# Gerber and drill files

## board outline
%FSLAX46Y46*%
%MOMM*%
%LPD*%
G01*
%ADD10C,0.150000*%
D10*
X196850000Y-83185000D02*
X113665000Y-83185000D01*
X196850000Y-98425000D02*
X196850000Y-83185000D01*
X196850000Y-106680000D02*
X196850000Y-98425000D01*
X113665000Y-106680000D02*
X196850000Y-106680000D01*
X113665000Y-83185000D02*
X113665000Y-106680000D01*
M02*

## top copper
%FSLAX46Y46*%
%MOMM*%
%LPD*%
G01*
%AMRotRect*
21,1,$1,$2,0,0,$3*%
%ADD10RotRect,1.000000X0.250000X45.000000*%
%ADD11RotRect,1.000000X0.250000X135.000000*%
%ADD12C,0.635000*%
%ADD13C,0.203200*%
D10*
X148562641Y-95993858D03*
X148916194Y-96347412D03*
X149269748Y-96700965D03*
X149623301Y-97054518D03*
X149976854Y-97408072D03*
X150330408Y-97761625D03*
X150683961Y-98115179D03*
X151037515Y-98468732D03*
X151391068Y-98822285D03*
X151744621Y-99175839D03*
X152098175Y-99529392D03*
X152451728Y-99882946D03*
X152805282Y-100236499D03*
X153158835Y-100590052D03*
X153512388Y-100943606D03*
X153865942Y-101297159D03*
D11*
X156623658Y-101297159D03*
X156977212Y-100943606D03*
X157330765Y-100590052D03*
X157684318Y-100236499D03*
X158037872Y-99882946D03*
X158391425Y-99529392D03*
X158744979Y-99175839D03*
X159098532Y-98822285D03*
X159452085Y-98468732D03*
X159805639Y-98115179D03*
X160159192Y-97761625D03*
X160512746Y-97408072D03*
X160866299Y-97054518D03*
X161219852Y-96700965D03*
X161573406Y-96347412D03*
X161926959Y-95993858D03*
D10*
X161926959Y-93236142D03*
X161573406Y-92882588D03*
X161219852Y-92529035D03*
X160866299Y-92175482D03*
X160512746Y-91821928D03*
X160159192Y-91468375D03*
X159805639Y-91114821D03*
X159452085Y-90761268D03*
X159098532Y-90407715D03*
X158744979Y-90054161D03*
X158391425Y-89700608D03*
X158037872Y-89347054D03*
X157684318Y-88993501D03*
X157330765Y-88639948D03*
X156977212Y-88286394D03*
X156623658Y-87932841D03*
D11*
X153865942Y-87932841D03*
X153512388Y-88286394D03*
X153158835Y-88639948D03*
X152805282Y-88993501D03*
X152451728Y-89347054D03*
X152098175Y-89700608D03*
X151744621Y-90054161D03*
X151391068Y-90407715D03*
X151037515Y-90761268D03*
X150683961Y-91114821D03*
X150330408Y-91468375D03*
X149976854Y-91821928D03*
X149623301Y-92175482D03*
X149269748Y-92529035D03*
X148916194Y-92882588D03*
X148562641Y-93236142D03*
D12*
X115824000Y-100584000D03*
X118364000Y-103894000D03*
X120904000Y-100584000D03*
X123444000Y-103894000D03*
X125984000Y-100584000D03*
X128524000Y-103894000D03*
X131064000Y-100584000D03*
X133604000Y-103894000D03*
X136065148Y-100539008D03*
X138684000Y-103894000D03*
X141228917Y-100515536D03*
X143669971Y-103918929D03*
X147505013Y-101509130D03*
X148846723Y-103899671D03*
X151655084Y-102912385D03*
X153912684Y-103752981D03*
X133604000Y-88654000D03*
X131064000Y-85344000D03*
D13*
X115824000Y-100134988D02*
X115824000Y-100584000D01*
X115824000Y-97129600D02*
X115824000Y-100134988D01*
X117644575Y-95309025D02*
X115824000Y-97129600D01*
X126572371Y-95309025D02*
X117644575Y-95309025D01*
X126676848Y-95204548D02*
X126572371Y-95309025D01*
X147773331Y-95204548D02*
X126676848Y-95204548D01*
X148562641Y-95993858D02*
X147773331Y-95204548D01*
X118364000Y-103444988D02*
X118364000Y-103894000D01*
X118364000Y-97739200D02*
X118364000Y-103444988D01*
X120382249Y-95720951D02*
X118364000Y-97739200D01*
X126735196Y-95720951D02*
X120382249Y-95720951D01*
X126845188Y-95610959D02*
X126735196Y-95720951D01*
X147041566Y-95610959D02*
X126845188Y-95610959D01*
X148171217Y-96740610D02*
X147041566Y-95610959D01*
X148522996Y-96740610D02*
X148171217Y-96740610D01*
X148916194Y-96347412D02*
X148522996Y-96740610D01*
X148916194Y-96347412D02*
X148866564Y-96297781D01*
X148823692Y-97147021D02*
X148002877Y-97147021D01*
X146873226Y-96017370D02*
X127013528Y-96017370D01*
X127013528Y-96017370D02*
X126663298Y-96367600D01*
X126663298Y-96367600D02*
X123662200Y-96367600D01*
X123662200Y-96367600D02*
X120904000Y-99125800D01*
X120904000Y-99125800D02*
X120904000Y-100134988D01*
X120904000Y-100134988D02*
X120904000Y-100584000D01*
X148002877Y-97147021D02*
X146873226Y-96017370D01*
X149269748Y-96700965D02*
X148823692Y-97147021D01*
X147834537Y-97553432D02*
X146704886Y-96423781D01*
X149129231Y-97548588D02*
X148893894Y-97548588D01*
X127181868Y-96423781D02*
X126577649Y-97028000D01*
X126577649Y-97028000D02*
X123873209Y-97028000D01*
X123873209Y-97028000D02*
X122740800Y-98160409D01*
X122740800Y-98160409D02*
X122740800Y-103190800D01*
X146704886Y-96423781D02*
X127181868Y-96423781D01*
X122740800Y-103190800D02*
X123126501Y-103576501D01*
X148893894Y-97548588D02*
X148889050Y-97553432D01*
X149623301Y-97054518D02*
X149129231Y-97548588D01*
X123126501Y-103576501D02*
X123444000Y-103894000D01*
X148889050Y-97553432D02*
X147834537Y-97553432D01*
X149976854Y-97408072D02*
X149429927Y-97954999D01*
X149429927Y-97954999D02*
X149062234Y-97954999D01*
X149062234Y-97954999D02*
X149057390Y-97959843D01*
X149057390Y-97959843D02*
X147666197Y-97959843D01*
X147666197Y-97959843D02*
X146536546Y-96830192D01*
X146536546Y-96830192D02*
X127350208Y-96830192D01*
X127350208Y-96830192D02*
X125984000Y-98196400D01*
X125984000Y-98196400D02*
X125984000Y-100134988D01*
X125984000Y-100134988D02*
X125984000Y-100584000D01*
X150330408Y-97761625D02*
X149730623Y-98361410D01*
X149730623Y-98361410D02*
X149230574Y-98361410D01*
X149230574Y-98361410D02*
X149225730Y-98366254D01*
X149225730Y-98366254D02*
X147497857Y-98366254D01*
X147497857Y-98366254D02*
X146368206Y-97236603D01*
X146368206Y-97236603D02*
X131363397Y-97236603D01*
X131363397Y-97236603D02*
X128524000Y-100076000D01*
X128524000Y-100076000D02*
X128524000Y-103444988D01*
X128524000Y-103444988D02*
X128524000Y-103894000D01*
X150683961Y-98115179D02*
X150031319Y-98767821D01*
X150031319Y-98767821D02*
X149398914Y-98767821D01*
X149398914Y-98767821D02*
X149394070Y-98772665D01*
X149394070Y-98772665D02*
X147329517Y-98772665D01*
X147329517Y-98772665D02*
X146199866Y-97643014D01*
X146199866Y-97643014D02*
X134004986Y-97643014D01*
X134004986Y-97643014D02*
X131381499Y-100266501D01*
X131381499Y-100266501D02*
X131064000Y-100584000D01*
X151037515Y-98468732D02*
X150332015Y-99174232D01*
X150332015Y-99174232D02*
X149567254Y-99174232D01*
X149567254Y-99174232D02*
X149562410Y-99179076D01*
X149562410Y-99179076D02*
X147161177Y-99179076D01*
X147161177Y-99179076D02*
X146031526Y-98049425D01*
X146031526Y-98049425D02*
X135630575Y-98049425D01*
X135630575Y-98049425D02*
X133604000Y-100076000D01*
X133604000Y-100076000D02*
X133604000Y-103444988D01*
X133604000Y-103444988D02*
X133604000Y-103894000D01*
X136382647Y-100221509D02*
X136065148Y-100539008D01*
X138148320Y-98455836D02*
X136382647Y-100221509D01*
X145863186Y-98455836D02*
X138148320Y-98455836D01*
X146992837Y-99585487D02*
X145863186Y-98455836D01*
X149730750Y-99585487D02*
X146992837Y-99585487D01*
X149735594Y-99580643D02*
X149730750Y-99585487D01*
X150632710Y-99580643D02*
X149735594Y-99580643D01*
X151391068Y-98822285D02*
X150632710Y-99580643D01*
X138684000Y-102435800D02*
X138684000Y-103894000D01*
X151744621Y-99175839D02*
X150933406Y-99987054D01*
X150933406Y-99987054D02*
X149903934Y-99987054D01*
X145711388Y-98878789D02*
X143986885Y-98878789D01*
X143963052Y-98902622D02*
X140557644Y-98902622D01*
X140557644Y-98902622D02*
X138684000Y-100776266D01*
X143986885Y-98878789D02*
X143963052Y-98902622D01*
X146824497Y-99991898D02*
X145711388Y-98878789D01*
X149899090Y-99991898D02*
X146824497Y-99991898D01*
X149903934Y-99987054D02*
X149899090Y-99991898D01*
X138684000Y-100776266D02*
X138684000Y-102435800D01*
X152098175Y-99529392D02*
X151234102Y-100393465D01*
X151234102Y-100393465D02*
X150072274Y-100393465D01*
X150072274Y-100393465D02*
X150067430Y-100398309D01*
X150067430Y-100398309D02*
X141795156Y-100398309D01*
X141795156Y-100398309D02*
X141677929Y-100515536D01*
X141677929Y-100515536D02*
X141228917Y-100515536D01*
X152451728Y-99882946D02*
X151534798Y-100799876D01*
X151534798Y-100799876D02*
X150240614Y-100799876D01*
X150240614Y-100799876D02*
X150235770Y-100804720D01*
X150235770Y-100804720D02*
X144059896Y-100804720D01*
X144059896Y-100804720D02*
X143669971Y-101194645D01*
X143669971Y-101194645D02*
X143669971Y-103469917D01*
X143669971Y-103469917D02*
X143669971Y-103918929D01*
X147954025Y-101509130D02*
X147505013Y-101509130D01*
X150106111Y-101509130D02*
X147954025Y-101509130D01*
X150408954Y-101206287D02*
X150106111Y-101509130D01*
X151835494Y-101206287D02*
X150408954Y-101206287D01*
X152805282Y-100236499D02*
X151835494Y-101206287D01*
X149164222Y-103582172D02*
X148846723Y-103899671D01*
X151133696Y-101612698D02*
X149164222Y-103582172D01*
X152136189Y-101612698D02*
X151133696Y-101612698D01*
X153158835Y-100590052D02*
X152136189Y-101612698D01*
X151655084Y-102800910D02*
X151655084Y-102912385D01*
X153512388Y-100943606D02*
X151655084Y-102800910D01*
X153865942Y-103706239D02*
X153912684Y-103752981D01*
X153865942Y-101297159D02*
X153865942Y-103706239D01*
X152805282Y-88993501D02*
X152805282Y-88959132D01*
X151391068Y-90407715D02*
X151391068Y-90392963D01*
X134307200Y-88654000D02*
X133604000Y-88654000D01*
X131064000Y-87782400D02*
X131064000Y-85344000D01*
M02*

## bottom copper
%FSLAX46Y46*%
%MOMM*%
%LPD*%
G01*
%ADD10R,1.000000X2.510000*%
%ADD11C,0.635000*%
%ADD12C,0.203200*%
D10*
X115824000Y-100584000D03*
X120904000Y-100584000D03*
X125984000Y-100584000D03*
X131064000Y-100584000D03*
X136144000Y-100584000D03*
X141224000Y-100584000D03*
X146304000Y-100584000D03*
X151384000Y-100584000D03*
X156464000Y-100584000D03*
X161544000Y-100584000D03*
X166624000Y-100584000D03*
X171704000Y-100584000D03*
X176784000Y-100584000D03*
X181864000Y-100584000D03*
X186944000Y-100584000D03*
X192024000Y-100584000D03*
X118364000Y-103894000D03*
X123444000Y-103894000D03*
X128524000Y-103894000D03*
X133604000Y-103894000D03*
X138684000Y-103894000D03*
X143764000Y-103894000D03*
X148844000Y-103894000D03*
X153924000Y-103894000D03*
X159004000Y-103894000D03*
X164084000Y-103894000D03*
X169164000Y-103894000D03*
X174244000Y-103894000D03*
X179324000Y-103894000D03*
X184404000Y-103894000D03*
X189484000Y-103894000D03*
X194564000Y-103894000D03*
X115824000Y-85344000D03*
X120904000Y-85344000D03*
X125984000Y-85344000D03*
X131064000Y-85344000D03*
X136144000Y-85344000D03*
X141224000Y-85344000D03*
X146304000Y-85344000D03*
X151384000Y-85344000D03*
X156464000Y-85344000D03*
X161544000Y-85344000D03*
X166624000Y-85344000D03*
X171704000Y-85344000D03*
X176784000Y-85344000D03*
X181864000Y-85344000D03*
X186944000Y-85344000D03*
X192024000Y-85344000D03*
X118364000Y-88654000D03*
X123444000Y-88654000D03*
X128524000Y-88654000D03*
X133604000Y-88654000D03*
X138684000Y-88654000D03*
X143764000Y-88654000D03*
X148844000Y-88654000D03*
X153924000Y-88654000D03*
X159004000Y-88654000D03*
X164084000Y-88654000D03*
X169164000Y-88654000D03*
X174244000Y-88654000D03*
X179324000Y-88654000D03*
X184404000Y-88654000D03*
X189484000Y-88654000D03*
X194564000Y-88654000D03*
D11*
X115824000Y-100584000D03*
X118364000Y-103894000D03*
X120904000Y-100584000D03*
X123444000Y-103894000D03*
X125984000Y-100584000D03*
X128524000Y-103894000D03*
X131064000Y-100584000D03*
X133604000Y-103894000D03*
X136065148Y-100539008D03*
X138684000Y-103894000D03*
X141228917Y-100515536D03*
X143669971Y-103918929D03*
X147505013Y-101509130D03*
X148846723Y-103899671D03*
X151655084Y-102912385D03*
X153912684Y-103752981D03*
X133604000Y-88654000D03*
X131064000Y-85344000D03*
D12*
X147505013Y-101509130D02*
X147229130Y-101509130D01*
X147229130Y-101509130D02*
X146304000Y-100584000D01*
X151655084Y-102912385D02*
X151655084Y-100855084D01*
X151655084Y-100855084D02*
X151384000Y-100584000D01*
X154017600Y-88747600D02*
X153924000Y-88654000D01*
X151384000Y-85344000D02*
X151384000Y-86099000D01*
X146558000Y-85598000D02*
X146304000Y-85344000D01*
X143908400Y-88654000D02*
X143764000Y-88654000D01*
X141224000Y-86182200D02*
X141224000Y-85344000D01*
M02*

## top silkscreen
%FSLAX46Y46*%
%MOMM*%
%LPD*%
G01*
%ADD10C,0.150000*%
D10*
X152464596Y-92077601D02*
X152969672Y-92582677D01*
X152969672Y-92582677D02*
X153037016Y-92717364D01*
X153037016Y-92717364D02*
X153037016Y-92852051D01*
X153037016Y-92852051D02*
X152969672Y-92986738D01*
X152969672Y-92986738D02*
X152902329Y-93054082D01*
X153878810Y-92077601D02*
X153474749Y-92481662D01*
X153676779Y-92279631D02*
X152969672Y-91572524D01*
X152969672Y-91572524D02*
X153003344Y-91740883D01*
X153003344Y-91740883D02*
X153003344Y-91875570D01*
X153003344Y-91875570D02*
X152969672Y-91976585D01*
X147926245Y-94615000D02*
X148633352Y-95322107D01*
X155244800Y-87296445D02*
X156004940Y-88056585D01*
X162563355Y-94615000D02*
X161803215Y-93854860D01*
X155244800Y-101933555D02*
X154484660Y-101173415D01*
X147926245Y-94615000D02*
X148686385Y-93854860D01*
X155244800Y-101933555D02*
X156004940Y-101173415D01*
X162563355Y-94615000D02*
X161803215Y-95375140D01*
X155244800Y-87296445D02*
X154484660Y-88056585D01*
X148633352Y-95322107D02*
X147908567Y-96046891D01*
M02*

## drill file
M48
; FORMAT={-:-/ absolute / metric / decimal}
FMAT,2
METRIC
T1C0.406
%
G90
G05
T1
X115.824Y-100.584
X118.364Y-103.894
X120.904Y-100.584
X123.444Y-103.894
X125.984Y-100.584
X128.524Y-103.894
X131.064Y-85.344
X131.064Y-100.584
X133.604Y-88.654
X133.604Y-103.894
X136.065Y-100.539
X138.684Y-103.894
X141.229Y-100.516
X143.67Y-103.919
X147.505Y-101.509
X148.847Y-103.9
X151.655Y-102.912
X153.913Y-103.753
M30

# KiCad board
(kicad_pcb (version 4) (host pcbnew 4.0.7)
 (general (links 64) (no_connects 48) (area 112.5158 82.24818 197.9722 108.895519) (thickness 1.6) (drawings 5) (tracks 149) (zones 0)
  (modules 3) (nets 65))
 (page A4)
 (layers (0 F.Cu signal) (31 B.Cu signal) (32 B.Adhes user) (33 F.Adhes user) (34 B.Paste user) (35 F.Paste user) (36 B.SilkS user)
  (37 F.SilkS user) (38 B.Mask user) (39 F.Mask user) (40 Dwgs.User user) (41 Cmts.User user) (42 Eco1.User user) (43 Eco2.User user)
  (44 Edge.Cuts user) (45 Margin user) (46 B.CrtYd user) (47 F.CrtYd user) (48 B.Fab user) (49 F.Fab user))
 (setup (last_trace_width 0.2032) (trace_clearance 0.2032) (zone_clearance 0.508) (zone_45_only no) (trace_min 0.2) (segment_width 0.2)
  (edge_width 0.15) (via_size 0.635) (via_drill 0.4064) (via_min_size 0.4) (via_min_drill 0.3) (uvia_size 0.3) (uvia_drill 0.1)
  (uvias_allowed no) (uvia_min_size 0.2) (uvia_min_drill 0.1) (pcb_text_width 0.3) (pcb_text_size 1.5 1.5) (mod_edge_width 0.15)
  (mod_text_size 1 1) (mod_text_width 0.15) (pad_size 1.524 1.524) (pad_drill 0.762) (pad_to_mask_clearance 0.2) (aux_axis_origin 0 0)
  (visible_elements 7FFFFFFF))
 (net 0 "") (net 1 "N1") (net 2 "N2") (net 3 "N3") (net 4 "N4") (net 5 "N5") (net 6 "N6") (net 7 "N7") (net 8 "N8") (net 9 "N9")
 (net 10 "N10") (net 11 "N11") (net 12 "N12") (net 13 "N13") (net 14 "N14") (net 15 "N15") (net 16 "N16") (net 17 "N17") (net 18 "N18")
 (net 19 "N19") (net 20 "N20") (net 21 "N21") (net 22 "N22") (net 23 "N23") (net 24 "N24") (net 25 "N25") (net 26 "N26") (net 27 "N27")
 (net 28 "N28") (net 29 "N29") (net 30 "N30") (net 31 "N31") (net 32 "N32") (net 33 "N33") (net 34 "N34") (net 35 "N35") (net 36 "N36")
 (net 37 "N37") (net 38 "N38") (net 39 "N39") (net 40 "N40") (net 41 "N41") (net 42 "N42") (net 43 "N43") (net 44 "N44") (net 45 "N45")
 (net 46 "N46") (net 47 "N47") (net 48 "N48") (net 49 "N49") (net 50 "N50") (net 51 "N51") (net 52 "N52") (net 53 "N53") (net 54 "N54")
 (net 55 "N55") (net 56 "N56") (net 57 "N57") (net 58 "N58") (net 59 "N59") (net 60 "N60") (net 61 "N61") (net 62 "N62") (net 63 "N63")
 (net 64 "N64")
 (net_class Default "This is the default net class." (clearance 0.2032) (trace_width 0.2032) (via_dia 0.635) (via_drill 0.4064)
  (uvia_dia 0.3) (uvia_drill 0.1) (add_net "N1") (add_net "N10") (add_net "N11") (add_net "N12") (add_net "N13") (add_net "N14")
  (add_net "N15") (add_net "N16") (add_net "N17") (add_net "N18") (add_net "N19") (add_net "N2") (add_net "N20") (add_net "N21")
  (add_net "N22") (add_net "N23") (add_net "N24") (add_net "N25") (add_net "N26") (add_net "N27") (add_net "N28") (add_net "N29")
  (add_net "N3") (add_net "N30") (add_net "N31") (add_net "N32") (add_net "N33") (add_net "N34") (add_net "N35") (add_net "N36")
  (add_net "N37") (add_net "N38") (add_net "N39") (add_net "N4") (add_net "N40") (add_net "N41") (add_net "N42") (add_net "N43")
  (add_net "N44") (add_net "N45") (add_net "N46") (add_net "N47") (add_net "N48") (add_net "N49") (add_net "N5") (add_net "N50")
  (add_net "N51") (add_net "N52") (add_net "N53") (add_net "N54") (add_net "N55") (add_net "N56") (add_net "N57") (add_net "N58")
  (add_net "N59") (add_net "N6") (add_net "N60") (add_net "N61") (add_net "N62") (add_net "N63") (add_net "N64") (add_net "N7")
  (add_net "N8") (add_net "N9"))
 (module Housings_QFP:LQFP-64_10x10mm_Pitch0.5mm (layer F.Cu) (at 155.2448 94.615 45)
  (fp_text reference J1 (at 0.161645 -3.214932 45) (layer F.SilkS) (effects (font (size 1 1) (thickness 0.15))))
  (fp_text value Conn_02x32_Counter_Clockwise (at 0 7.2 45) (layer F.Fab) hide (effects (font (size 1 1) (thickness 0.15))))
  (fp_line (start -5.175 -5.175) (end -5.175 -4.175) (layer F.SilkS) (width 0.15))
  (fp_line (start 5.175 -5.175) (end 5.175 -4.1) (layer F.SilkS) (width 0.15))
  (fp_line (start 5.175 5.175) (end 5.175 4.1) (layer F.SilkS) (width 0.15))
  (fp_line (start -5.175 5.175) (end -5.175 4.1) (layer F.SilkS) (width 0.15))
  (fp_line (start -5.175 -5.175) (end -4.1 -5.175) (layer F.SilkS) (width 0.15))
  (fp_line (start -5.175 5.175) (end -4.1 5.175) (layer F.SilkS) (width 0.15))
  (fp_line (start 5.175 5.175) (end 4.1 5.175) (layer F.SilkS) (width 0.15))
  (fp_line (start 5.175 -5.175) (end 4.1 -5.175) (layer F.SilkS) (width 0.15))
  (fp_line (start -5.175 -4.175) (end -6.2 -4.175) (layer F.SilkS) (width 0.15))
  (pad 1 smd rect (at -5.7 -3.75 45) (size 1 0.25) (layers F.Cu F.Paste F.Mask) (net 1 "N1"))
  (pad 2 smd rect (at -5.7 -3.25 45) (size 1 0.25) (layers F.Cu F.Paste F.Mask) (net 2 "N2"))
  (pad 3 smd rect (at -5.7 -2.75 45) (size 1 0.25) (layers F.Cu F.Paste F.Mask) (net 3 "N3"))
  (pad 4 smd rect (at -5.7 -2.25 45) (size 1 0.25) (layers F.Cu F.Paste F.Mask) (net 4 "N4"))
  (pad 5 smd rect (at -5.7 -1.75 45) (size 1 0.25) (layers F.Cu F.Paste F.Mask) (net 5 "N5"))
  (pad 6 smd rect (at -5.7 -1.25 45) (size 1 0.25) (layers F.Cu F.Paste F.Mask) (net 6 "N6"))
  (pad 7 smd rect (at -5.7 -0.75 45) (size 1 0.25) (layers F.Cu F.Paste F.Mask) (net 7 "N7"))
  (pad 8 smd rect (at -5.7 -0.25 45) (size 1 0.25) (layers F.Cu F.Paste F.Mask) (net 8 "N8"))
  (pad 9 smd rect (at -5.7 0.25 45) (size 1 0.25) (layers F.Cu F.Paste F.Mask) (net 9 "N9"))
  (pad 10 smd rect (at -5.7 0.75 45) (size 1 0.25) (layers F.Cu F.Paste F.Mask) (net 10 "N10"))
  (pad 11 smd rect (at -5.7 1.25 45) (size 1 0.25) (layers F.Cu F.Paste F.Mask) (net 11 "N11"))
  (pad 12 smd rect (at -5.7 1.75 45) (size 1 0.25) (layers F.Cu F.Paste F.Mask) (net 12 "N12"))
  (pad 13 smd rect (at -5.7 2.25 45) (size 1 0.25) (layers F.Cu F.Paste F.Mask) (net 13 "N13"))
  (pad 14 smd rect (at -5.7 2.75 45) (size 1 0.25) (layers F.Cu F.Paste F.Mask) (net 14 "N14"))
  (pad 15 smd rect (at -5.7 3.25 45) (size 1 0.25) (layers F.Cu F.Paste F.Mask) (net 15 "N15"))
  (pad 16 smd rect (at -5.7 3.75 45) (size 1 0.25) (layers F.Cu F.Paste F.Mask) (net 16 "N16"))
  (pad 17 smd rect (at -3.75 5.7 135) (size 1 0.25) (layers F.Cu F.Paste F.Mask) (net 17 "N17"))
  (pad 18 smd rect (at -3.25 5.7 135) (size 1 0.25) (layers F.Cu F.Paste F.Mask) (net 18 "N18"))
  (pad 19 smd rect (at -2.75 5.7 135) (size 1 0.25) (layers F.Cu F.Paste F.Mask) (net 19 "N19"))
  (pad 20 smd rect (at -2.25 5.7 135) (size 1 0.25) (layers F.Cu F.Paste F.Mask) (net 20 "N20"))
  (pad 21 smd rect (at -1.75 5.7 135) (size 1 0.25) (layers F.Cu F.Paste F.Mask) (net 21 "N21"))
  (pad 22 smd rect (at -1.25 5.7 135) (size 1 0.25) (layers F.Cu F.Paste F.Mask) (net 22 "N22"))
  (pad 23 smd rect (at -0.75 5.7 135) (size 1 0.25) (layers F.Cu F.Paste F.Mask) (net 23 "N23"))
  (pad 24 smd rect (at -0.25 5.7 135) (size 1 0.25) (layers F.Cu F.Paste F.Mask) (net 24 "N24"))
  (pad 25 smd rect (at 0.25 5.7 135) (size 1 0.25) (layers F.Cu F.Paste F.Mask) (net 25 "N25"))
  (pad 26 smd rect (at 0.75 5.7 135) (size 1 0.25) (layers F.Cu F.Paste F.Mask) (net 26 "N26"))
  (pad 27 smd rect (at 1.25 5.7 135) (size 1 0.25) (layers F.Cu F.Paste F.Mask) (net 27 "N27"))
  (pad 28 smd rect (at 1.75 5.7 135) (size 1 0.25) (layers F.Cu F.Paste F.Mask) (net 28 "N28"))
  (pad 29 smd rect (at 2.25 5.7 135) (size 1 0.25) (layers F.Cu F.Paste F.Mask) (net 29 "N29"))
  (pad 30 smd rect (at 2.75 5.7 135) (size 1 0.25) (layers F.Cu F.Paste F.Mask) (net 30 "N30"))
  (pad 31 smd rect (at 3.25 5.7 135) (size 1 0.25) (layers F.Cu F.Paste F.Mask) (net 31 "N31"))
  (pad 32 smd rect (at 3.75 5.7 135) (size 1 0.25) (layers F.Cu F.Paste F.Mask) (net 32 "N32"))
  (pad 33 smd rect (at 5.7 3.75 45) (size 1 0.25) (layers F.Cu F.Paste F.Mask) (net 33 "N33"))
  (pad 34 smd rect (at 5.7 3.25 45) (size 1 0.25) (layers F.Cu F.Paste F.Mask) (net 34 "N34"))
  (pad 35 smd rect (at 5.7 2.75 45) (size 1 0.25) (layers F.Cu F.Paste F.Mask) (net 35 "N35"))
  (pad 36 smd rect (at 5.7 2.25 45) (size 1 0.25) (layers F.Cu F.Paste F.Mask) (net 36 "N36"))
  (pad 37 smd rect (at 5.7 1.75 45) (size 1 0.25) (layers F.Cu F.Paste F.Mask) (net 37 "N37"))
  (pad 38 smd rect (at 5.7 1.25 45) (size 1 0.25) (layers F.Cu F.Paste F.Mask) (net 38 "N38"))
  (pad 39 smd rect (at 5.7 0.75 45) (size 1 0.25) (layers F.Cu F.Paste F.Mask) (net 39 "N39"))
  (pad 40 smd rect (at 5.7 0.25 45) (size 1 0.25) (layers F.Cu F.Paste F.Mask) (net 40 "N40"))
  (pad 41 smd rect (at 5.7 -0.25 45) (size 1 0.25) (layers F.Cu F.Paste F.Mask) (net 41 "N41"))
  (pad 42 smd rect (at 5.7 -0.75 45) (size 1 0.25) (layers F.Cu F.Paste F.Mask) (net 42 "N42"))
  (pad 43 smd rect (at 5.7 -1.25 45) (size 1 0.25) (layers F.Cu F.Paste F.Mask) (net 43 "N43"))
  (pad 44 smd rect (at 5.7 -1.75 45) (size 1 0.25) (layers F.Cu F.Paste F.Mask) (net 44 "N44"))
  (pad 45 smd rect (at 5.7 -2.25 45) (size 1 0.25) (layers F.Cu F.Paste F.Mask) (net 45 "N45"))
  (pad 46 smd rect (at 5.7 -2.75 45) (size 1 0.25) (layers F.Cu F.Paste F.Mask) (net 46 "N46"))
  (pad 47 smd rect (at 5.7 -3.25 45) (size 1 0.25) (layers F.Cu F.Paste F.Mask) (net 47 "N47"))
  (pad 48 smd rect (at 5.7 -3.75 45) (size 1 0.25) (layers F.Cu F.Paste F.Mask) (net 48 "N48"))
  (pad 49 smd rect (at 3.75 -5.7 135) (size 1 0.25) (layers F.Cu F.Paste F.Mask) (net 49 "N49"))
  (pad 50 smd rect (at 3.25 -5.7 135) (size 1 0.25) (layers F.Cu F.Paste F.Mask) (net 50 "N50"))
  (pad 51 smd rect (at 2.75 -5.7 135) (size 1 0.25) (layers F.Cu F.Paste F.Mask) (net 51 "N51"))
  (pad 52 smd rect (at 2.25 -5.7 135) (size 1 0.25) (layers F.Cu F.Paste F.Mask) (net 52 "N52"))
  (pad 53 smd rect (at 1.75 -5.7 135) (size 1 0.25) (layers F.Cu F.Paste F.Mask) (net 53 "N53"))
  (pad 54 smd rect (at 1.25 -5.7 135) (size 1 0.25) (layers F.Cu F.Paste F.Mask) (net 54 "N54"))
  (pad 55 smd rect (at 0.75 -5.7 135) (size 1 0.25) (layers F.Cu F.Paste F.Mask) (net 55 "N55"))
  (pad 56 smd rect (at 0.25 -5.7 135) (size 1 0.25) (layers F.Cu F.Paste F.Mask) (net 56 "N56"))
  (pad 57 smd rect (at -0.25 -5.7 135) (size 1 0.25) (layers F.Cu F.Paste F.Mask) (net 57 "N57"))
  (pad 58 smd rect (at -0.75 -5.7 135) (size 1 0.25) (layers F.Cu F.Paste F.Mask) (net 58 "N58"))
  (pad 59 smd rect (at -1.25 -5.7 135) (size 1 0.25) (layers F.Cu F.Paste F.Mask) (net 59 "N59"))
  (pad 60 smd rect (at -1.75 -5.7 135) (size 1 0.25) (layers F.Cu F.Paste F.Mask) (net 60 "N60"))
  (pad 61 smd rect (at -2.25 -5.7 135) (size 1 0.25) (layers F.Cu F.Paste F.Mask) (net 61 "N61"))
  (pad 62 smd rect (at -2.75 -5.7 135) (size 1 0.25) (layers F.Cu F.Paste F.Mask) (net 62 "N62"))
  (pad 63 smd rect (at -3.25 -5.7 135) (size 1 0.25) (layers F.Cu F.Paste F.Mask) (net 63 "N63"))
  (pad 64 smd rect (at -3.75 -5.7 135) (size 1 0.25) (layers F.Cu F.Paste F.Mask) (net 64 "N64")))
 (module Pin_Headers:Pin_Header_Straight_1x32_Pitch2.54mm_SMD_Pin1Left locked (layer B.Cu) (at 155.194 102.239 270)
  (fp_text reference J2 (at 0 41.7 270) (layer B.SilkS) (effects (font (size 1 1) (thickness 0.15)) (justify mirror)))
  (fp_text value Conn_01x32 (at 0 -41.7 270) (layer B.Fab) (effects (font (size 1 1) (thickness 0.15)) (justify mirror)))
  (pad 1 smd rect (at -1.655 39.37 270) (size 2.51 1) (layers B.Cu B.Paste B.Mask) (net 1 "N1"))
  (pad 3 smd rect (at -1.655 34.29 270) (size 2.51 1) (layers B.Cu B.Paste B.Mask) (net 3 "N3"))
  (pad 5 smd rect (at -1.655 29.21 270) (size 2.51 1) (layers B.Cu B.Paste B.Mask) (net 5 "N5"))
  (pad 7 smd rect (at -1.655 24.13 270) (size 2.51 1) (layers B.Cu B.Paste B.Mask) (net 7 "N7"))
  (pad 9 smd rect (at -1.655 19.05 270) (size 2.51 1) (layers B.Cu B.Paste B.Mask) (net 9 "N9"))
  (pad 11 smd rect (at -1.655 13.97 270) (size 2.51 1) (layers B.Cu B.Paste B.Mask) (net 11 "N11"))
  (pad 13 smd rect (at -1.655 8.89 270) (size 2.51 1) (layers B.Cu B.Paste B.Mask) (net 13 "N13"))
  (pad 15 smd rect (at -1.655 3.81 270) (size 2.51 1) (layers B.Cu B.Paste B.Mask) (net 15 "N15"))
  (pad 17 smd rect (at -1.655 -1.27 270) (size 2.51 1) (layers B.Cu B.Paste B.Mask) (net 17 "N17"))
  (pad 19 smd rect (at -1.655 -6.35 270) (size 2.51 1) (layers B.Cu B.Paste B.Mask) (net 19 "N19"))
  (pad 21 smd rect (at -1.655 -11.43 270) (size 2.51 1) (layers B.Cu B.Paste B.Mask) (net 21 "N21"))
  (pad 23 smd rect (at -1.655 -16.51 270) (size 2.51 1) (layers B.Cu B.Paste B.Mask) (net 23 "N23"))
  (pad 25 smd rect (at -1.655 -21.59 270) (size 2.51 1) (layers B.Cu B.Paste B.Mask) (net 25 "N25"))
  (pad 27 smd rect (at -1.655 -26.67 270) (size 2.51 1) (layers B.Cu B.Paste B.Mask) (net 27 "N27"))
  (pad 29 smd rect (at -1.655 -31.75 270) (size 2.51 1) (layers B.Cu B.Paste B.Mask) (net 29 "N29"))
  (pad 31 smd rect (at -1.655 -36.83 270) (size 2.51 1) (layers B.Cu B.Paste B.Mask) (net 31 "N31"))
  (pad 2 smd rect (at 1.655 36.83 270) (size 2.51 1) (layers B.Cu B.Paste B.Mask) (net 2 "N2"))
  (pad 4 smd rect (at 1.655 31.75 270) (size 2.51 1) (layers B.Cu B.Paste B.Mask) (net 4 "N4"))
  (pad 6 smd rect (at 1.655 26.67 270) (size 2.51 1) (layers B.Cu B.Paste B.Mask) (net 6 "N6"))
  (pad 8 smd rect (at 1.655 21.59 270) (size 2.51 1) (layers B.Cu B.Paste B.Mask) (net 8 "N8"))
  (pad 10 smd rect (at 1.655 16.51 270) (size 2.51 1) (layers B.Cu B.Paste B.Mask) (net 10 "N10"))
  (pad 12 smd rect (at 1.655 11.43 270) (size 2.51 1) (layers B.Cu B.Paste B.Mask) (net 12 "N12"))
  (pad 14 smd rect (at 1.655 6.35 270) (size 2.51 1) (layers B.Cu B.Paste B.Mask) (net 14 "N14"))
  (pad 16 smd rect (at 1.655 1.27 270) (size 2.51 1) (layers B.Cu B.Paste B.Mask) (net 16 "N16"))
  (pad 18 smd rect (at 1.655 -3.81 270) (size 2.51 1) (layers B.Cu B.Paste B.Mask) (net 18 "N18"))
  (pad 20 smd rect (at 1.655 -8.89 270) (size 2.51 1) (layers B.Cu B.Paste B.Mask) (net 20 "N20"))
  (pad 22 smd rect (at 1.655 -13.97 270) (size 2.51 1) (layers B.Cu B.Paste B.Mask) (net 22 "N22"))
  (pad 24 smd rect (at 1.655 -19.05 270) (size 2.51 1) (layers B.Cu B.Paste B.Mask) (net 24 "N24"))
  (pad 26 smd rect (at 1.655 -24.13 270) (size 2.51 1) (layers B.Cu B.Paste B.Mask) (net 26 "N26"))
  (pad 28 smd rect (at 1.655 -29.21 270) (size 2.51 1) (layers B.Cu B.Paste B.Mask) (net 28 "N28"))
  (pad 30 smd rect (at 1.655 -34.29 270) (size 2.51 1) (layers B.Cu B.Paste B.Mask) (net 30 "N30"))
  (pad 32 smd rect (at 1.655 -39.37 270) (size 2.51 1) (layers B.Cu B.Paste B.Mask) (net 32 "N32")))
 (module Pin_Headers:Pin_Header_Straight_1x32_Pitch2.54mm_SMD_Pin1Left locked (layer B.Cu) (at 155.194 86.999 270)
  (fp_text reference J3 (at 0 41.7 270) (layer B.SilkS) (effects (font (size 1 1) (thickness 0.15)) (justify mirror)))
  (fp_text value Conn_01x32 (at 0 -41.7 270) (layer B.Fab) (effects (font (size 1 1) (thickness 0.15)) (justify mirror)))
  (pad 1 smd rect (at -1.655 39.37 270) (size 2.51 1) (layers B.Cu B.Paste B.Mask) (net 64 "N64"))
  (pad 3 smd rect (at -1.655 34.29 270) (size 2.51 1) (layers B.Cu B.Paste B.Mask) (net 62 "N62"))
  (pad 5 smd rect (at -1.655 29.21 270) (size 2.51 1) (layers B.Cu B.Paste B.Mask) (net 60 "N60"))
  (pad 7 smd rect (at -1.655 24.13 270) (size 2.51 1) (layers B.Cu B.Paste B.Mask) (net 58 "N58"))
  (pad 9 smd rect (at -1.655 19.05 270) (size 2.51 1) (layers B.Cu B.Paste B.Mask) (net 56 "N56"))
  (pad 11 smd rect (at -1.655 13.97 270) (size 2.51 1) (layers B.Cu B.Paste B.Mask) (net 54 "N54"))
  (pad 13 smd rect (at -1.655 8.89 270) (size 2.51 1) (layers B.Cu B.Paste B.Mask) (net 52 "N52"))
  (pad 15 smd rect (at -1.655 3.81 270) (size 2.51 1) (layers B.Cu B.Paste B.Mask) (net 50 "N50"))
  (pad 17 smd rect (at -1.655 -1.27 270) (size 2.51 1) (layers B.Cu B.Paste B.Mask) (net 48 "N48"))
  (pad 19 smd rect (at -1.655 -6.35 270) (size 2.51 1) (layers B.Cu B.Paste B.Mask) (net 46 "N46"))
  (pad 21 smd rect (at -1.655 -11.43 270) (size 2.51 1) (layers B.Cu B.Paste B.Mask) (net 44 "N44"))
  (pad 23 smd rect (at -1.655 -16.51 270) (size 2.51 1) (layers B.Cu B.Paste B.Mask) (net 42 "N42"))
  (pad 25 smd rect (at -1.655 -21.59 270) (size 2.51 1) (layers B.Cu B.Paste B.Mask) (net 40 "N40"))
  (pad 27 smd rect (at -1.655 -26.67 270) (size 2.51 1) (layers B.Cu B.Paste B.Mask) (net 38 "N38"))
  (pad 29 smd rect (at -1.655 -31.75 270) (size 2.51 1) (layers B.Cu B.Paste B.Mask) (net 36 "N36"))
  (pad 31 smd rect (at -1.655 -36.83 270) (size 2.51 1) (layers B.Cu B.Paste B.Mask) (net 34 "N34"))
  (pad 2 smd rect (at 1.655 36.83 270) (size 2.51 1) (layers B.Cu B.Paste B.Mask) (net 63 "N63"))
  (pad 4 smd rect (at 1.655 31.75 270) (size 2.51 1) (layers B.Cu B.Paste B.Mask) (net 61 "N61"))
  (pad 6 smd rect (at 1.655 26.67 270) (size 2.51 1) (layers B.Cu B.Paste B.Mask) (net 59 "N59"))
  (pad 8 smd rect (at 1.655 21.59 270) (size 2.51 1) (layers B.Cu B.Paste B.Mask) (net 57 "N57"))
  (pad 10 smd rect (at 1.655 16.51 270) (size 2.51 1) (layers B.Cu B.Paste B.Mask) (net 55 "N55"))
  (pad 12 smd rect (at 1.655 11.43 270) (size 2.51 1) (layers B.Cu B.Paste B.Mask) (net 53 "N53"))
  (pad 14 smd rect (at 1.655 6.35 270) (size 2.51 1) (layers B.Cu B.Paste B.Mask) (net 51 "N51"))
  (pad 16 smd rect (at 1.655 1.27 270) (size 2.51 1) (layers B.Cu B.Paste B.Mask) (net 49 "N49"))
  (pad 18 smd rect (at 1.655 -3.81 270) (size 2.51 1) (layers B.Cu B.Paste B.Mask) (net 47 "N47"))
  (pad 20 smd rect (at 1.655 -8.89 270) (size 2.51 1) (layers B.Cu B.Paste B.Mask) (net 45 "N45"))
  (pad 22 smd rect (at 1.655 -13.97 270) (size 2.51 1) (layers B.Cu B.Paste B.Mask) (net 43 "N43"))
  (pad 24 smd rect (at 1.655 -19.05 270) (size 2.51 1) (layers B.Cu B.Paste B.Mask) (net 41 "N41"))
  (pad 26 smd rect (at 1.655 -24.13 270) (size 2.51 1) (layers B.Cu B.Paste B.Mask) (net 39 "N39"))
  (pad 28 smd rect (at 1.655 -29.21 270) (size 2.51 1) (layers B.Cu B.Paste B.Mask) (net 37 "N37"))
  (pad 30 smd rect (at 1.655 -34.29 270) (size 2.51 1) (layers B.Cu B.Paste B.Mask) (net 35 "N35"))
  (pad 32 smd rect (at 1.655 -39.37 270) (size 2.51 1) (layers B.Cu B.Paste B.Mask) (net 33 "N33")))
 (gr_line (start 196.85 83.185) (end 113.665 83.185) (angle 90) (layer Edge.Cuts) (width 0.15))
 (gr_line (start 196.85 98.425) (end 196.85 83.185) (angle 90) (layer Edge.Cuts) (width 0.15))
 (gr_line (start 196.85 106.68) (end 196.85 98.425) (angle 90) (layer Edge.Cuts) (width 0.15))
 (gr_line (start 113.665 106.68) (end 196.85 106.68) (angle 90) (layer Edge.Cuts) (width 0.15))
 (gr_line (start 113.665 83.185) (end 113.665 106.68) (angle 90) (layer Edge.Cuts) (width 0.15))
 (segment (start 115.824 100.134988) (end 115.824 100.584) (width 0.2032) (layer F.Cu) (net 1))
 (segment (start 115.824 97.1296) (end 115.824 100.134988) (width 0.2032) (layer F.Cu) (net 1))
 (segment (start 117.644575 95.309025) (end 115.824 97.1296) (width 0.2032) (layer F.Cu) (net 1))
 (segment (start 126.572371 95.309025) (end 117.644575 95.309025) (width 0.2032) (layer F.Cu) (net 1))
 (segment (start 126.676848 95.204548) (end 126.572371 95.309025) (width 0.2032) (layer F.Cu) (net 1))
 (segment (start 147.773331 95.204548) (end 126.676848 95.204548) (width 0.2032) (layer F.Cu) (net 1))
 (segment (start 148.562641 95.993858) (end 147.773331 95.204548) (width 0.2032) (layer F.Cu) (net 1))
 (via (at 115.824 100.584) (size 0.635) (drill 0.4064) (layers F.Cu B.Cu) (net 1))
 (segment (start 118.364 103.444988) (end 118.364 103.894) (width 0.2032) (layer F.Cu) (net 2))
 (segment (start 118.364 97.7392) (end 118.364 103.444988) (width 0.2032) (layer F.Cu) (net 2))
 (segment (start 120.382249 95.720951) (end 118.364 97.7392) (width 0.2032) (layer F.Cu) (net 2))
 (segment (start 126.735196 95.720951) (end 120.382249 95.720951) (width 0.2032) (layer F.Cu) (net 2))
 (segment (start 126.845188 95.610959) (end 126.735196 95.720951) (width 0.2032) (layer F.Cu) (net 2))
 (segment (start 147.041566 95.610959) (end 126.845188 95.610959) (width 0.2032) (layer F.Cu) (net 2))
 (segment (start 148.171217 96.74061) (end 147.041566 95.610959) (width 0.2032) (layer F.Cu) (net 2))
 (segment (start 148.522996 96.74061) (end 148.171217 96.74061) (width 0.2032) (layer F.Cu) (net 2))
 (segment (start 148.916194 96.347412) (end 148.522996 96.74061) (width 0.2032) (layer F.Cu) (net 2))
 (segment (start 148.916194 96.347412) (end 148.866564 96.297781) (width 0.2032) (layer F.Cu) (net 2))
 (via (at 118.364 103.894) (size 0.635) (drill 0.4064) (layers F.Cu B.Cu) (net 2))
 (segment (start 148.823692 97.147021) (end 148.002877 97.147021) (width 0.2032) (layer F.Cu) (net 3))
 (segment (start 146.873226 96.01737) (end 127.013528 96.01737) (width 0.2032) (layer F.Cu) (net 3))
 (segment (start 127.013528 96.01737) (end 126.663298 96.3676) (width 0.2032) (layer F.Cu) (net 3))
 (segment (start 126.663298 96.3676) (end 123.6622 96.3676) (width 0.2032) (layer F.Cu) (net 3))
 (segment (start 123.6622 96.3676) (end 120.904 99.1258) (width 0.2032) (layer F.Cu) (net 3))
 (segment (start 120.904 99.1258) (end 120.904 100.134988) (width 0.2032) (layer F.Cu) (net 3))
 (segment (start 120.904 100.134988) (end 120.904 100.584) (width 0.2032) (layer F.Cu) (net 3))
 (segment (start 148.002877 97.147021) (end 146.873226 96.01737) (width 0.2032) (layer F.Cu) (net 3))
 (segment (start 149.269748 96.700965) (end 148.823692 97.147021) (width 0.2032) (layer F.Cu) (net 3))
 (via (at 120.904 100.584) (size 0.635) (drill 0.4064) (layers F.Cu B.Cu) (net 3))
 (segment (start 147.834537 97.553432) (end 146.704886 96.423781) (width 0.2032) (layer F.Cu) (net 4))
 (segment (start 149.129231 97.548588) (end 148.893894 97.548588) (width 0.2032) (layer F.Cu) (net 4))
 (segment (start 127.181868 96.423781) (end 126.577649 97.028) (width 0.2032) (layer F.Cu) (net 4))
 (segment (start 126.577649 97.028) (end 123.873209 97.028) (width 0.2032) (layer F.Cu) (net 4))
 (segment (start 123.873209 97.028) (end 122.7408 98.160409) (width 0.2032) (layer F.Cu) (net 4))
 (segment (start 122.7408 98.160409) (end 122.7408 103.1908) (width 0.2032) (layer F.Cu) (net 4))
 (segment (start 146.704886 96.423781) (end 127.181868 96.423781) (width 0.2032) (layer F.Cu) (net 4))
 (segment (start 122.7408 103.1908) (end 123.126501 103.576501) (width 0.2032) (layer F.Cu) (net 4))
 (segment (start 148.893894 97.548588) (end 148.88905 97.553432) (width 0.2032) (layer F.Cu) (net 4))
 (segment (start 149.623301 97.054518) (end 149.129231 97.548588) (width 0.2032) (layer F.Cu) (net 4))
 (segment (start 123.126501 103.576501) (end 123.444 103.894) (width 0.2032) (layer F.Cu) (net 4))
 (segment (start 148.88905 97.553432) (end 147.834537 97.553432) (width 0.2032) (layer F.Cu) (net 4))
 (via (at 123.444 103.894) (size 0.635) (drill 0.4064) (layers F.Cu B.Cu) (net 4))
 (segment (start 149.976854 97.408072) (end 149.429927 97.954999) (width 0.2032) (layer F.Cu) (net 5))
 (segment (start 149.429927 97.954999) (end 149.062234 97.954999) (width 0.2032) (layer F.Cu) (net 5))
 (segment (start 149.062234 97.954999) (end 149.05739 97.959843) (width 0.2032) (layer F.Cu) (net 5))
 (segment (start 149.05739 97.959843) (end 147.666197 97.959843) (width 0.2032) (layer F.Cu) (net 5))
 (segment (start 147.666197 97.959843) (end 146.536546 96.830192) (width 0.2032) (layer F.Cu) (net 5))
 (segment (start 146.536546 96.830192) (end 127.350208 96.830192) (width 0.2032) (layer F.Cu) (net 5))
 (segment (start 127.350208 96.830192) (end 125.984 98.1964) (width 0.2032) (layer F.Cu) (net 5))
 (segment (start 125.984 98.1964) (end 125.984 100.134988) (width 0.2032) (layer F.Cu) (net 5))
 (segment (start 125.984 100.134988) (end 125.984 100.584) (width 0.2032) (layer F.Cu) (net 5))
 (via (at 125.984 100.584) (size 0.635) (drill 0.4064) (layers F.Cu B.Cu) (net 5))
 (segment (start 150.330408 97.761625) (end 149.730623 98.36141) (width 0.2032) (layer F.Cu) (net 6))
 (segment (start 149.730623 98.36141) (end 149.230574 98.36141) (width 0.2032) (layer F.Cu) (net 6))
 (segment (start 149.230574 98.36141) (end 149.22573 98.366254) (width 0.2032) (layer F.Cu) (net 6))
 (segment (start 149.22573 98.366254) (end 147.497857 98.366254) (width 0.2032) (layer F.Cu) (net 6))
 (segment (start 147.497857 98.366254) (end 146.368206 97.236603) (width 0.2032) (layer F.Cu) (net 6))
 (segment (start 146.368206 97.236603) (end 131.363397 97.236603) (width 0.2032) (layer F.Cu) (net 6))
 (segment (start 131.363397 97.236603) (end 128.524 100.076) (width 0.2032) (layer F.Cu) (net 6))
 (segment (start 128.524 100.076) (end 128.524 103.444988) (width 0.2032) (layer F.Cu) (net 6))
 (segment (start 128.524 103.444988) (end 128.524 103.894) (width 0.2032) (layer F.Cu) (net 6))
 (via (at 128.524 103.894) (size 0.635) (drill 0.4064) (layers F.Cu B.Cu) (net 6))
 (segment (start 150.683961 98.115179) (end 150.031319 98.767821) (width 0.2032) (layer F.Cu) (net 7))
 (segment (start 150.031319 98.767821) (end 149.398914 98.767821) (width 0.2032) (layer F.Cu) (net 7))
 (segment (start 149.398914 98.767821) (end 149.39407 98.772665) (width 0.2032) (layer F.Cu) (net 7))
 (segment (start 149.39407 98.772665) (end 147.329517 98.772665) (width 0.2032) (layer F.Cu) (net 7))
 (segment (start 147.329517 98.772665) (end 146.199866 97.643014) (width 0.2032) (layer F.Cu) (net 7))
 (segment (start 146.199866 97.643014) (end 134.004986 97.643014) (width 0.2032) (layer F.Cu) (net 7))
 (segment (start 134.004986 97.643014) (end 131.381499 100.266501) (width 0.2032) (layer F.Cu) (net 7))
 (segment (start 131.381499 100.266501) (end 131.064 100.584) (width 0.2032) (layer F.Cu) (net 7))
 (via (at 131.064 100.584) (size 0.635) (drill 0.4064) (layers F.Cu B.Cu) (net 7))
 (segment (start 151.037515 98.468732) (end 150.332015 99.174232) (width 0.2032) (layer F.Cu) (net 8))
 (segment (start 150.332015 99.174232) (end 149.567254 99.174232) (width 0.2032) (layer F.Cu) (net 8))
 (segment (start 149.567254 99.174232) (end 149.56241 99.179076) (width 0.2032) (layer F.Cu) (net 8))
 (segment (start 149.56241 99.179076) (end 147.161177 99.179076) (width 0.2032) (layer F.Cu) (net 8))
 (segment (start 147.161177 99.179076) (end 146.031526 98.049425) (width 0.2032) (layer F.Cu) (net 8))
 (segment (start 146.031526 98.049425) (end 135.630575 98.049425) (width 0.2032) (layer F.Cu) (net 8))
 (segment (start 135.630575 98.049425) (end 133.604 100.076) (width 0.2032) (layer F.Cu) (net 8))
 (segment (start 133.604 100.076) (end 133.604 103.444988) (width 0.2032) (layer F.Cu) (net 8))
 (segment (start 133.604 103.444988) (end 133.604 103.894) (width 0.2032) (layer F.Cu) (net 8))
 (via (at 133.604 103.894) (size 0.635) (drill 0.4064) (layers F.Cu B.Cu) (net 8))
 (segment (start 136.382647 100.221509) (end 136.065148 100.539008) (width 0.2032) (layer F.Cu) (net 9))
 (segment (start 138.14832 98.455836) (end 136.382647 100.221509) (width 0.2032) (layer F.Cu) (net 9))
 (segment (start 145.863186 98.455836) (end 138.14832 98.455836) (width 0.2032) (layer F.Cu) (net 9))
 (segment (start 146.992837 99.585487) (end 145.863186 98.455836) (width 0.2032) (layer F.Cu) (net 9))
 (segment (start 149.73075 99.585487) (end 146.992837 99.585487) (width 0.2032) (layer F.Cu) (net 9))
 (segment (start 149.735594 99.580643) (end 149.73075 99.585487) (width 0.2032) (layer F.Cu) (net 9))
 (segment (start 150.63271 99.580643) (end 149.735594 99.580643) (width 0.2032) (layer F.Cu) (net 9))
 (segment (start 151.391068 98.822285) (end 150.63271 99.580643) (width 0.2032) (layer F.Cu) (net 9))
 (via (at 136.065148 100.539008) (size 0.635) (drill 0.4064) (layers F.Cu B.Cu) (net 9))
 (segment (start 138.684 102.4358) (end 138.684 103.894) (width 0.2032) (layer F.Cu) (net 10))
 (segment (start 151.744621 99.175839) (end 150.933406 99.987054) (width 0.2032) (layer F.Cu) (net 10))
 (segment (start 150.933406 99.987054) (end 149.903934 99.987054) (width 0.2032) (layer F.Cu) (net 10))
 (segment (start 145.711388 98.878789) (end 143.986885 98.878789) (width 0.2032) (layer F.Cu) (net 10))
 (segment (start 143.963052 98.902622) (end 140.557644 98.902622) (width 0.2032) (layer F.Cu) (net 10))
 (segment (start 140.557644 98.902622) (end 138.684 100.776266) (width 0.2032) (layer F.Cu) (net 10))
 (segment (start 143.986885 98.878789) (end 143.963052 98.902622) (width 0.2032) (layer F.Cu) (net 10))
 (segment (start 146.824497 99.991898) (end 145.711388 98.878789) (width 0.2032) (layer F.Cu) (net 10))
 (segment (start 149.89909 99.991898) (end 146.824497 99.991898) (width 0.2032) (layer F.Cu) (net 10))
 (segment (start 149.903934 99.987054) (end 149.89909 99.991898) (width 0.2032) (layer F.Cu) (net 10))
 (segment (start 138.684 100.776266) (end 138.684 102.4358) (width 0.2032) (layer F.Cu) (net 10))
 (via (at 138.684 103.894) (size 0.635) (drill 0.4064) (layers F.Cu B.Cu) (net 10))
 (segment (start 152.098175 99.529392) (end 151.234102 100.393465) (width 0.2032) (layer F.Cu) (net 11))
 (segment (start 151.234102 100.393465) (end 150.072274 100.393465) (width 0.2032) (layer F.Cu) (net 11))
 (segment (start 150.072274 100.393465) (end 150.06743 100.398309) (width 0.2032) (layer F.Cu) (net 11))
 (segment (start 150.06743 100.398309) (end 141.795156 100.398309) (width 0.2032) (layer F.Cu) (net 11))
 (segment (start 141.795156 100.398309) (end 141.677929 100.515536) (width 0.2032) (layer F.Cu) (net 11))
 (segment (start 141.677929 100.515536) (end 141.228917 100.515536) (width 0.2032) (layer F.Cu) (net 11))
 (via (at 141.228917 100.515536) (size 0.635) (drill 0.4064) (layers F.Cu B.Cu) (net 11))
 (segment (start 152.451728 99.882946) (end 151.534798 100.799876) (width 0.2032) (layer F.Cu) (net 12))
 (segment (start 151.534798 100.799876) (end 150.240614 100.799876) (width 0.2032) (layer F.Cu) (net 12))
 (segment (start 150.240614 100.799876) (end 150.23577 100.80472) (width 0.2032) (layer F.Cu) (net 12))
 (segment (start 150.23577 100.80472) (end 144.059896 100.80472) (width 0.2032) (layer F.Cu) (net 12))
 (segment (start 144.059896 100.80472) (end 143.669971 101.194645) (width 0.2032) (layer F.Cu) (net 12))
 (segment (start 143.669971 101.194645) (end 143.669971 103.469917) (width 0.2032) (layer F.Cu) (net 12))
 (segment (start 143.669971 103.469917) (end 143.669971 103.918929) (width 0.2032) (layer F.Cu) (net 12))
 (via (at 143.669971 103.918929) (size 0.635) (drill 0.4064) (layers F.Cu B.Cu) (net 12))
 (segment (start 147.505013 101.50913) (end 147.22913 101.50913) (width 0.2032) (layer B.Cu) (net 13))
 (segment (start 147.22913 101.50913) (end 146.304 100.584) (width 0.2032) (layer B.Cu) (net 13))
 (segment (start 147.954025 101.50913) (end 147.505013 101.50913) (width 0.2032) (layer F.Cu) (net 13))
 (segment (start 150.106111 101.50913) (end 147.954025 101.50913) (width 0.2032) (layer F.Cu) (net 13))
 (segment (start 150.408954 101.206287) (end 150.106111 101.50913) (width 0.2032) (layer F.Cu) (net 13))
 (segment (start 151.835494 101.206287) (end 150.408954 101.206287) (width 0.2032) (layer F.Cu) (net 13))
 (segment (start 152.805282 100.236499) (end 151.835494 101.206287) (width 0.2032) (layer F.Cu) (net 13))
 (via (at 147.505013 101.50913) (size 0.635) (drill 0.4064) (layers F.Cu B.Cu) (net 13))
 (segment (start 149.164222 103.582172) (end 148.846723 103.899671) (width 0.2032) (layer F.Cu) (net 14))
 (segment (start 151.133696 101.612698) (end 149.164222 103.582172) (width 0.2032) (layer F.Cu) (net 14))
 (segment (start 152.136189 101.612698) (end 151.133696 101.612698) (width 0.2032) (layer F.Cu) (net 14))
 (segment (start 153.158835 100.590052) (end 152.136189 101.612698) (width 0.2032) (layer F.Cu) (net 14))
 (via (at 148.846723 103.899671) (size 0.635) (drill 0.4064) (layers F.Cu B.Cu) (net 14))
 (segment (start 151.655084 102.912385) (end 151.655084 100.855084) (width 0.2032) (layer B.Cu) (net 15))
 (segment (start 151.655084 100.855084) (end 151.384 100.584) (width 0.2032) (layer B.Cu) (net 15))
 (segment (start 151.655084 102.80091) (end 151.655084 102.912385) (width 0.2032) (layer F.Cu) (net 15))
 (segment (start 153.512388 100.943606) (end 151.655084 102.80091) (width 0.2032) (layer F.Cu) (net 15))
 (via (at 151.655084 102.912385) (size 0.635) (drill 0.4064) (layers F.Cu B.Cu) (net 15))
 (segment (start 153.865942 103.706239) (end 153.912684 103.752981) (width 0.2032) (layer F.Cu) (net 16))
 (segment (start 153.865942 101.297159) (end 153.865942 103.706239) (width 0.2032) (layer F.Cu) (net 16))
 (via (at 153.912684 103.752981) (size 0.635) (drill 0.4064) (layers F.Cu B.Cu) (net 16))
 (segment (start 154.0176 88.7476) (end 153.924 88.654) (width 0.2032) (layer B.Cu) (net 49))
 (segment (start 151.384 85.344) (end 151.384 86.099) (width 0.2032) (layer B.Cu) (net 50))
 (segment (start 152.805282 88.993501) (end 152.805282 88.959132) (width 0.2032) (layer F.Cu) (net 52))
 (segment (start 146.558 85.598) (end 146.304 85.344) (width 0.2032) (layer B.Cu) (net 52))
 (segment (start 143.9084 88.654) (end 143.764 88.654) (width 0.2032) (layer B.Cu) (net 53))
 (segment (start 141.224 86.1822) (end 141.224 85.344) (width 0.2032) (layer B.Cu) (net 54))
 (segment (start 151.391068 90.407715) (end 151.391068 90.392963) (width 0.2032) (layer F.Cu) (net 56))
 (segment (start 134.3072 88.654) (end 133.604 88.654) (width 0.2032) (layer F.Cu) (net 57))
 (via (at 133.604 88.654) (size 0.635) (drill 0.4064) (layers F.Cu B.Cu) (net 57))
 (segment (start 131.064 87.7824) (end 131.064 85.344) (width 0.2032) (layer F.Cu) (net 58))
 (via (at 131.064 85.344) (size 0.635) (drill 0.4064) (layers F.Cu B.Cu) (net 58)))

